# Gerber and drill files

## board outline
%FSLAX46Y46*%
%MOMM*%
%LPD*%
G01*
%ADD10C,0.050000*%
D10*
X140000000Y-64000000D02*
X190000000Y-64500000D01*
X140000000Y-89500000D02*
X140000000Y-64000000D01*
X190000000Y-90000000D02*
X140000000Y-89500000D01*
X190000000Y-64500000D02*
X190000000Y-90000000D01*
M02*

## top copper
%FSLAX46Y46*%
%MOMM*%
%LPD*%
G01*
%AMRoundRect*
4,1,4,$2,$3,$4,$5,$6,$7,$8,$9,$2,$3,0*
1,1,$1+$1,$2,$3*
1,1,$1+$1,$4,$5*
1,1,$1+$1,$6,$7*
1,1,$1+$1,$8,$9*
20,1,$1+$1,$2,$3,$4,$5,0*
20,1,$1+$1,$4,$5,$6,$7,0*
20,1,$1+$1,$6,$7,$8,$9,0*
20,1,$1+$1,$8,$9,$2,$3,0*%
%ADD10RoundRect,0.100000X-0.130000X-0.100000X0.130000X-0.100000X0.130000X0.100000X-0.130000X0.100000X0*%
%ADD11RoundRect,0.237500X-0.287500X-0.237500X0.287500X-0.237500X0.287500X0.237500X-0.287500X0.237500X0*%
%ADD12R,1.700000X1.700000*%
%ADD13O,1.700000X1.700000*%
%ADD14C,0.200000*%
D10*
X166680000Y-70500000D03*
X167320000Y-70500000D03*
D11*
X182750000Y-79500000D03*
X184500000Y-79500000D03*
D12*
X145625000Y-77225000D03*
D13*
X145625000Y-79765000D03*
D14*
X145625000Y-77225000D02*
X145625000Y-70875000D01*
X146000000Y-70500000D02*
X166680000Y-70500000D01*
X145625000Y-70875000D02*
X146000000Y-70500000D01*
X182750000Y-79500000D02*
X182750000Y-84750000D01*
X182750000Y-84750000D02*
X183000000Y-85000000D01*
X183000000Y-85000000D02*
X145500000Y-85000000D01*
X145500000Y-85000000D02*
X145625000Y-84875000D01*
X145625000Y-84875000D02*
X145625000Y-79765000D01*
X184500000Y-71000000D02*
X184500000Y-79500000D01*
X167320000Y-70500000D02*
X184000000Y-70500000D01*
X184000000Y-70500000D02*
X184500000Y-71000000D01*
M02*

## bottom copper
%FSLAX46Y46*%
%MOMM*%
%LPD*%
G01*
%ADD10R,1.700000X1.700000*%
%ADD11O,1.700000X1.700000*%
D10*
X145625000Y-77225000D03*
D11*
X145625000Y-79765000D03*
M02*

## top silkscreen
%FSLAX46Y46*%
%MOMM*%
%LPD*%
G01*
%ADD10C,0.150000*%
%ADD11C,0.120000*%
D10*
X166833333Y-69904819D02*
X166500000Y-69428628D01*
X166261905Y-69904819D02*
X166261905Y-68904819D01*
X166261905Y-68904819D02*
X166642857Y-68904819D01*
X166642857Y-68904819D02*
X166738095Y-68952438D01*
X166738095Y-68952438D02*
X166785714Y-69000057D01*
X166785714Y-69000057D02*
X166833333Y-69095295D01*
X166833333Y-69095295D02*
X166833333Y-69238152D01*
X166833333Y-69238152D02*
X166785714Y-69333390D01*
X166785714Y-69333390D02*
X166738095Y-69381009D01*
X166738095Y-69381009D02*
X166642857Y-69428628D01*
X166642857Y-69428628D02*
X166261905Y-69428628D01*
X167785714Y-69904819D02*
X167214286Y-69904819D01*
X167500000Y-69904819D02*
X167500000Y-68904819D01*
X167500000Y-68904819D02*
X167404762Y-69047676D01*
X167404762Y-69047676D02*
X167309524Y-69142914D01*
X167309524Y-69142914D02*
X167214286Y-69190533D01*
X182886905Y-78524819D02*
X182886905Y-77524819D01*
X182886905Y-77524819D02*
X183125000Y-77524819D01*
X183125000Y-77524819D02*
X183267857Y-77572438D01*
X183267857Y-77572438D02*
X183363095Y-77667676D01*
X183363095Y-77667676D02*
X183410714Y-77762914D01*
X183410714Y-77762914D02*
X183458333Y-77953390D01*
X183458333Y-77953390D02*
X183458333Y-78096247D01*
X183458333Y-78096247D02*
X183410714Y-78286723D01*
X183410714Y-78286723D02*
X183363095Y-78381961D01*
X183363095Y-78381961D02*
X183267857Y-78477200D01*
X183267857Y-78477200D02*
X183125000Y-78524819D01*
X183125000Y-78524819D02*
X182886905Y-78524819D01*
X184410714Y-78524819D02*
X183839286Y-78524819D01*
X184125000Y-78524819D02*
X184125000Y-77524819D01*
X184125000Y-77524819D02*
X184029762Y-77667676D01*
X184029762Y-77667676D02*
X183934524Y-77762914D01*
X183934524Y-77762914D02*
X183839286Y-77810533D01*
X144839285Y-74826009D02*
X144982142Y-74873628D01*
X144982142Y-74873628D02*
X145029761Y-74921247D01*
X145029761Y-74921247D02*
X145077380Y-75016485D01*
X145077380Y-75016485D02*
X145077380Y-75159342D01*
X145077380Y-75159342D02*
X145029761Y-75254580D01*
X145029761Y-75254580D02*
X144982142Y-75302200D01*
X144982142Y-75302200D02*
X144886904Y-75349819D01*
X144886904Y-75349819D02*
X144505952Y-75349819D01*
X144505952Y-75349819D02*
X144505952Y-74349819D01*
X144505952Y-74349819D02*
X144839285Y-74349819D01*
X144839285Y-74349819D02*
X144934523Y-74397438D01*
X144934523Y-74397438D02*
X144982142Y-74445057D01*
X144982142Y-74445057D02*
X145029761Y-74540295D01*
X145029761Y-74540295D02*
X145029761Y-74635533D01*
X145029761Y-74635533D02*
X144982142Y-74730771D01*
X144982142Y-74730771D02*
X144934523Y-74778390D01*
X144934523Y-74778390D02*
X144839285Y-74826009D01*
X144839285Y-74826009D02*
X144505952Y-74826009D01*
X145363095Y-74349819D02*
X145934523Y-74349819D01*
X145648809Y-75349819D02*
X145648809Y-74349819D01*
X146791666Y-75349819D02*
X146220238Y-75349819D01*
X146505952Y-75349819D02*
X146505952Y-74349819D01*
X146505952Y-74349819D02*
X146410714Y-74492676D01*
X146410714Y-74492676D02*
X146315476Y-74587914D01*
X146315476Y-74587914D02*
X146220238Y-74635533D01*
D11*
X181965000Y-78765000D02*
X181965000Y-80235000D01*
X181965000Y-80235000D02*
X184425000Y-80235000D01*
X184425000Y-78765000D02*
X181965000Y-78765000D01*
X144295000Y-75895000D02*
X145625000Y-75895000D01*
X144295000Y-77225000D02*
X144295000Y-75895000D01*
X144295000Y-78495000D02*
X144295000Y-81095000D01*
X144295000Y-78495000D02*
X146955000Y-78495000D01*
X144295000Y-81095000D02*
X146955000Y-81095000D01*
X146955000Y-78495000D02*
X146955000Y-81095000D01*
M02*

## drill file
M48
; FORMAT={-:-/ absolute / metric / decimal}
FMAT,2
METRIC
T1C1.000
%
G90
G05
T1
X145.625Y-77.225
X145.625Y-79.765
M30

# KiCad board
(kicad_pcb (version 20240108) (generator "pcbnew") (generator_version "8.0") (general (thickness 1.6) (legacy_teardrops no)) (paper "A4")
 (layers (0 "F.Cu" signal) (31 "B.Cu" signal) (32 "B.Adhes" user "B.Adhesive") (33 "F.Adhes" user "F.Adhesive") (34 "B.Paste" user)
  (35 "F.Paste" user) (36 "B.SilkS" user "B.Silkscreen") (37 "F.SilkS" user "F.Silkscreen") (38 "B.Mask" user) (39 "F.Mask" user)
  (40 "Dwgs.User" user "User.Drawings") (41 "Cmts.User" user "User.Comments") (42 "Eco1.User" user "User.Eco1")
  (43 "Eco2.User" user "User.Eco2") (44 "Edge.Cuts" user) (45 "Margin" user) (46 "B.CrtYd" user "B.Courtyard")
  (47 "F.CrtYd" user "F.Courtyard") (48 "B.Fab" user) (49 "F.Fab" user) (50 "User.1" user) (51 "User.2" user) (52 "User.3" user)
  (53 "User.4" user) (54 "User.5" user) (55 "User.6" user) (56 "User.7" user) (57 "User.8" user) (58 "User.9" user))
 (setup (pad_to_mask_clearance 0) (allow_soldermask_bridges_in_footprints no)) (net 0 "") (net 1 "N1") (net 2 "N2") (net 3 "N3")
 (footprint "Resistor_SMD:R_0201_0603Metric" (layer "F.Cu") (at 167 70.5)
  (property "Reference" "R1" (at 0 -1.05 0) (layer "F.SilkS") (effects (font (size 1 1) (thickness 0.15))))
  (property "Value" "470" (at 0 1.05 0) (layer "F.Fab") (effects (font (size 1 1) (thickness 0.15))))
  (pad "" smd roundrect (at -0.345 0) (size 0.318 0.36) (layers "F.Paste") (roundrect_rratio 0.25))
  (pad "" smd roundrect (at 0.345 0) (size 0.318 0.36) (layers "F.Paste") (roundrect_rratio 0.25))
  (pad "1" smd roundrect (at -0.32 0) (size 0.46 0.4) (layers "F.Cu" "F.Mask") (roundrect_rratio 0.25) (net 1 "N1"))
  (pad "2" smd roundrect (at 0.32 0) (size 0.46 0.4) (layers "F.Cu" "F.Mask") (roundrect_rratio 0.25) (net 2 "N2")))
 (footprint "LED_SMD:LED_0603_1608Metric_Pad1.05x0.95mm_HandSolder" (layer "F.Cu") (at 183.625 79.5)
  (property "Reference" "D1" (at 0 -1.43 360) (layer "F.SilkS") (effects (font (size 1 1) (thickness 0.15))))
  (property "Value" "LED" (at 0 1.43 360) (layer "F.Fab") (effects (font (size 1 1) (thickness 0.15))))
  (fp_line (start -1.66 -0.735) (end -1.66 0.735) (stroke (width 0.12) (type solid)) (layer "F.SilkS"))
  (fp_line (start -1.66 0.735) (end 0.8 0.735) (stroke (width 0.12) (type solid)) (layer "F.SilkS"))
  (fp_line (start 0.8 -0.735) (end -1.66 -0.735) (stroke (width 0.12) (type solid)) (layer "F.SilkS"))
  (pad "1" smd roundrect (at -0.875 0) (size 1.05 0.95) (layers "F.Cu" "F.Paste" "F.Mask") (roundrect_rratio 0.25) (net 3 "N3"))
  (pad "2" smd roundrect (at 0.875 0) (size 1.05 0.95) (layers "F.Cu" "F.Paste" "F.Mask") (roundrect_rratio 0.25) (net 2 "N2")))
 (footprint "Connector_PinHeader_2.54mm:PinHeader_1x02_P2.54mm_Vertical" (layer "F.Cu") (at 145.625 77.225)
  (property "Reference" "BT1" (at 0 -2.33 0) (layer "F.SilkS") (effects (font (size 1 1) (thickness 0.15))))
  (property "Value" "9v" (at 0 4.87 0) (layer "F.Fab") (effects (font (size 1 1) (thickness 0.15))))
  (fp_line (start -1.33 -1.33) (end 0 -1.33) (stroke (width 0.12) (type solid)) (layer "F.SilkS"))
  (fp_line (start -1.33 0) (end -1.33 -1.33) (stroke (width 0.12) (type solid)) (layer "F.SilkS"))
  (fp_line (start -1.33 1.27) (end -1.33 3.87) (stroke (width 0.12) (type solid)) (layer "F.SilkS"))
  (fp_line (start -1.33 1.27) (end 1.33 1.27) (stroke (width 0.12) (type solid)) (layer "F.SilkS"))
  (fp_line (start -1.33 3.87) (end 1.33 3.87) (stroke (width 0.12) (type solid)) (layer "F.SilkS"))
  (fp_line (start 1.33 1.27) (end 1.33 3.87) (stroke (width 0.12) (type solid)) (layer "F.SilkS"))
  (pad "1" thru_hole rect (at 0 0) (size 1.7 1.7) (drill 1) (layers "*.Cu" "*.Mask") (remove_unused_layers no) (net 1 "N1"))
  (pad "2" thru_hole oval (at 0 2.54) (size 1.7 1.7) (drill 1) (layers "*.Cu" "*.Mask") (remove_unused_layers no) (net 3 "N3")))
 (gr_line (start 140 64) (end 190 64.5) (stroke (width 0.05) (type default)) (layer "Edge.Cuts"))
 (gr_line (start 140 89.5) (end 140 64) (stroke (width 0.05) (type default)) (layer "Edge.Cuts"))
 (gr_line (start 190 90) (end 140 89.5) (stroke (width 0.05) (type default)) (layer "Edge.Cuts"))
 (gr_line (start 190 64.5) (end 190 90) (stroke (width 0.05) (type default)) (layer "Edge.Cuts"))
 (segment (start 145.625 77.225) (end 145.625 70.875) (width 0.2) (layer "F.Cu") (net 1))
 (segment (start 146 70.5) (end 166.68 70.5) (width 0.2) (layer "F.Cu") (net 1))
 (segment (start 145.625 70.875) (end 146 70.5) (width 0.2) (layer "F.Cu") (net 1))
 (segment (start 182.75 79.5) (end 182.75 84.75) (width 0.2) (layer "F.Cu") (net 3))
 (segment (start 182.75 84.75) (end 183 85) (width 0.2) (layer "F.Cu") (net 3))
 (segment (start 183 85) (end 145.5 85) (width 0.2) (layer "F.Cu") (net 3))
 (segment (start 145.5 85) (end 145.625 84.875) (width 0.2) (layer "F.Cu") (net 3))
 (segment (start 145.625 84.875) (end 145.625 79.765) (width 0.2) (layer "F.Cu") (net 3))
 (segment (start 184.5 71) (end 184.5 79.5) (width 0.2) (layer "F.Cu") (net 2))
 (segment (start 167.32 70.5) (end 184 70.5) (width 0.2) (layer "F.Cu") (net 2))
 (segment (start 184 70.5) (end 184.5 71) (width 0.2) (layer "F.Cu") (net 2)))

